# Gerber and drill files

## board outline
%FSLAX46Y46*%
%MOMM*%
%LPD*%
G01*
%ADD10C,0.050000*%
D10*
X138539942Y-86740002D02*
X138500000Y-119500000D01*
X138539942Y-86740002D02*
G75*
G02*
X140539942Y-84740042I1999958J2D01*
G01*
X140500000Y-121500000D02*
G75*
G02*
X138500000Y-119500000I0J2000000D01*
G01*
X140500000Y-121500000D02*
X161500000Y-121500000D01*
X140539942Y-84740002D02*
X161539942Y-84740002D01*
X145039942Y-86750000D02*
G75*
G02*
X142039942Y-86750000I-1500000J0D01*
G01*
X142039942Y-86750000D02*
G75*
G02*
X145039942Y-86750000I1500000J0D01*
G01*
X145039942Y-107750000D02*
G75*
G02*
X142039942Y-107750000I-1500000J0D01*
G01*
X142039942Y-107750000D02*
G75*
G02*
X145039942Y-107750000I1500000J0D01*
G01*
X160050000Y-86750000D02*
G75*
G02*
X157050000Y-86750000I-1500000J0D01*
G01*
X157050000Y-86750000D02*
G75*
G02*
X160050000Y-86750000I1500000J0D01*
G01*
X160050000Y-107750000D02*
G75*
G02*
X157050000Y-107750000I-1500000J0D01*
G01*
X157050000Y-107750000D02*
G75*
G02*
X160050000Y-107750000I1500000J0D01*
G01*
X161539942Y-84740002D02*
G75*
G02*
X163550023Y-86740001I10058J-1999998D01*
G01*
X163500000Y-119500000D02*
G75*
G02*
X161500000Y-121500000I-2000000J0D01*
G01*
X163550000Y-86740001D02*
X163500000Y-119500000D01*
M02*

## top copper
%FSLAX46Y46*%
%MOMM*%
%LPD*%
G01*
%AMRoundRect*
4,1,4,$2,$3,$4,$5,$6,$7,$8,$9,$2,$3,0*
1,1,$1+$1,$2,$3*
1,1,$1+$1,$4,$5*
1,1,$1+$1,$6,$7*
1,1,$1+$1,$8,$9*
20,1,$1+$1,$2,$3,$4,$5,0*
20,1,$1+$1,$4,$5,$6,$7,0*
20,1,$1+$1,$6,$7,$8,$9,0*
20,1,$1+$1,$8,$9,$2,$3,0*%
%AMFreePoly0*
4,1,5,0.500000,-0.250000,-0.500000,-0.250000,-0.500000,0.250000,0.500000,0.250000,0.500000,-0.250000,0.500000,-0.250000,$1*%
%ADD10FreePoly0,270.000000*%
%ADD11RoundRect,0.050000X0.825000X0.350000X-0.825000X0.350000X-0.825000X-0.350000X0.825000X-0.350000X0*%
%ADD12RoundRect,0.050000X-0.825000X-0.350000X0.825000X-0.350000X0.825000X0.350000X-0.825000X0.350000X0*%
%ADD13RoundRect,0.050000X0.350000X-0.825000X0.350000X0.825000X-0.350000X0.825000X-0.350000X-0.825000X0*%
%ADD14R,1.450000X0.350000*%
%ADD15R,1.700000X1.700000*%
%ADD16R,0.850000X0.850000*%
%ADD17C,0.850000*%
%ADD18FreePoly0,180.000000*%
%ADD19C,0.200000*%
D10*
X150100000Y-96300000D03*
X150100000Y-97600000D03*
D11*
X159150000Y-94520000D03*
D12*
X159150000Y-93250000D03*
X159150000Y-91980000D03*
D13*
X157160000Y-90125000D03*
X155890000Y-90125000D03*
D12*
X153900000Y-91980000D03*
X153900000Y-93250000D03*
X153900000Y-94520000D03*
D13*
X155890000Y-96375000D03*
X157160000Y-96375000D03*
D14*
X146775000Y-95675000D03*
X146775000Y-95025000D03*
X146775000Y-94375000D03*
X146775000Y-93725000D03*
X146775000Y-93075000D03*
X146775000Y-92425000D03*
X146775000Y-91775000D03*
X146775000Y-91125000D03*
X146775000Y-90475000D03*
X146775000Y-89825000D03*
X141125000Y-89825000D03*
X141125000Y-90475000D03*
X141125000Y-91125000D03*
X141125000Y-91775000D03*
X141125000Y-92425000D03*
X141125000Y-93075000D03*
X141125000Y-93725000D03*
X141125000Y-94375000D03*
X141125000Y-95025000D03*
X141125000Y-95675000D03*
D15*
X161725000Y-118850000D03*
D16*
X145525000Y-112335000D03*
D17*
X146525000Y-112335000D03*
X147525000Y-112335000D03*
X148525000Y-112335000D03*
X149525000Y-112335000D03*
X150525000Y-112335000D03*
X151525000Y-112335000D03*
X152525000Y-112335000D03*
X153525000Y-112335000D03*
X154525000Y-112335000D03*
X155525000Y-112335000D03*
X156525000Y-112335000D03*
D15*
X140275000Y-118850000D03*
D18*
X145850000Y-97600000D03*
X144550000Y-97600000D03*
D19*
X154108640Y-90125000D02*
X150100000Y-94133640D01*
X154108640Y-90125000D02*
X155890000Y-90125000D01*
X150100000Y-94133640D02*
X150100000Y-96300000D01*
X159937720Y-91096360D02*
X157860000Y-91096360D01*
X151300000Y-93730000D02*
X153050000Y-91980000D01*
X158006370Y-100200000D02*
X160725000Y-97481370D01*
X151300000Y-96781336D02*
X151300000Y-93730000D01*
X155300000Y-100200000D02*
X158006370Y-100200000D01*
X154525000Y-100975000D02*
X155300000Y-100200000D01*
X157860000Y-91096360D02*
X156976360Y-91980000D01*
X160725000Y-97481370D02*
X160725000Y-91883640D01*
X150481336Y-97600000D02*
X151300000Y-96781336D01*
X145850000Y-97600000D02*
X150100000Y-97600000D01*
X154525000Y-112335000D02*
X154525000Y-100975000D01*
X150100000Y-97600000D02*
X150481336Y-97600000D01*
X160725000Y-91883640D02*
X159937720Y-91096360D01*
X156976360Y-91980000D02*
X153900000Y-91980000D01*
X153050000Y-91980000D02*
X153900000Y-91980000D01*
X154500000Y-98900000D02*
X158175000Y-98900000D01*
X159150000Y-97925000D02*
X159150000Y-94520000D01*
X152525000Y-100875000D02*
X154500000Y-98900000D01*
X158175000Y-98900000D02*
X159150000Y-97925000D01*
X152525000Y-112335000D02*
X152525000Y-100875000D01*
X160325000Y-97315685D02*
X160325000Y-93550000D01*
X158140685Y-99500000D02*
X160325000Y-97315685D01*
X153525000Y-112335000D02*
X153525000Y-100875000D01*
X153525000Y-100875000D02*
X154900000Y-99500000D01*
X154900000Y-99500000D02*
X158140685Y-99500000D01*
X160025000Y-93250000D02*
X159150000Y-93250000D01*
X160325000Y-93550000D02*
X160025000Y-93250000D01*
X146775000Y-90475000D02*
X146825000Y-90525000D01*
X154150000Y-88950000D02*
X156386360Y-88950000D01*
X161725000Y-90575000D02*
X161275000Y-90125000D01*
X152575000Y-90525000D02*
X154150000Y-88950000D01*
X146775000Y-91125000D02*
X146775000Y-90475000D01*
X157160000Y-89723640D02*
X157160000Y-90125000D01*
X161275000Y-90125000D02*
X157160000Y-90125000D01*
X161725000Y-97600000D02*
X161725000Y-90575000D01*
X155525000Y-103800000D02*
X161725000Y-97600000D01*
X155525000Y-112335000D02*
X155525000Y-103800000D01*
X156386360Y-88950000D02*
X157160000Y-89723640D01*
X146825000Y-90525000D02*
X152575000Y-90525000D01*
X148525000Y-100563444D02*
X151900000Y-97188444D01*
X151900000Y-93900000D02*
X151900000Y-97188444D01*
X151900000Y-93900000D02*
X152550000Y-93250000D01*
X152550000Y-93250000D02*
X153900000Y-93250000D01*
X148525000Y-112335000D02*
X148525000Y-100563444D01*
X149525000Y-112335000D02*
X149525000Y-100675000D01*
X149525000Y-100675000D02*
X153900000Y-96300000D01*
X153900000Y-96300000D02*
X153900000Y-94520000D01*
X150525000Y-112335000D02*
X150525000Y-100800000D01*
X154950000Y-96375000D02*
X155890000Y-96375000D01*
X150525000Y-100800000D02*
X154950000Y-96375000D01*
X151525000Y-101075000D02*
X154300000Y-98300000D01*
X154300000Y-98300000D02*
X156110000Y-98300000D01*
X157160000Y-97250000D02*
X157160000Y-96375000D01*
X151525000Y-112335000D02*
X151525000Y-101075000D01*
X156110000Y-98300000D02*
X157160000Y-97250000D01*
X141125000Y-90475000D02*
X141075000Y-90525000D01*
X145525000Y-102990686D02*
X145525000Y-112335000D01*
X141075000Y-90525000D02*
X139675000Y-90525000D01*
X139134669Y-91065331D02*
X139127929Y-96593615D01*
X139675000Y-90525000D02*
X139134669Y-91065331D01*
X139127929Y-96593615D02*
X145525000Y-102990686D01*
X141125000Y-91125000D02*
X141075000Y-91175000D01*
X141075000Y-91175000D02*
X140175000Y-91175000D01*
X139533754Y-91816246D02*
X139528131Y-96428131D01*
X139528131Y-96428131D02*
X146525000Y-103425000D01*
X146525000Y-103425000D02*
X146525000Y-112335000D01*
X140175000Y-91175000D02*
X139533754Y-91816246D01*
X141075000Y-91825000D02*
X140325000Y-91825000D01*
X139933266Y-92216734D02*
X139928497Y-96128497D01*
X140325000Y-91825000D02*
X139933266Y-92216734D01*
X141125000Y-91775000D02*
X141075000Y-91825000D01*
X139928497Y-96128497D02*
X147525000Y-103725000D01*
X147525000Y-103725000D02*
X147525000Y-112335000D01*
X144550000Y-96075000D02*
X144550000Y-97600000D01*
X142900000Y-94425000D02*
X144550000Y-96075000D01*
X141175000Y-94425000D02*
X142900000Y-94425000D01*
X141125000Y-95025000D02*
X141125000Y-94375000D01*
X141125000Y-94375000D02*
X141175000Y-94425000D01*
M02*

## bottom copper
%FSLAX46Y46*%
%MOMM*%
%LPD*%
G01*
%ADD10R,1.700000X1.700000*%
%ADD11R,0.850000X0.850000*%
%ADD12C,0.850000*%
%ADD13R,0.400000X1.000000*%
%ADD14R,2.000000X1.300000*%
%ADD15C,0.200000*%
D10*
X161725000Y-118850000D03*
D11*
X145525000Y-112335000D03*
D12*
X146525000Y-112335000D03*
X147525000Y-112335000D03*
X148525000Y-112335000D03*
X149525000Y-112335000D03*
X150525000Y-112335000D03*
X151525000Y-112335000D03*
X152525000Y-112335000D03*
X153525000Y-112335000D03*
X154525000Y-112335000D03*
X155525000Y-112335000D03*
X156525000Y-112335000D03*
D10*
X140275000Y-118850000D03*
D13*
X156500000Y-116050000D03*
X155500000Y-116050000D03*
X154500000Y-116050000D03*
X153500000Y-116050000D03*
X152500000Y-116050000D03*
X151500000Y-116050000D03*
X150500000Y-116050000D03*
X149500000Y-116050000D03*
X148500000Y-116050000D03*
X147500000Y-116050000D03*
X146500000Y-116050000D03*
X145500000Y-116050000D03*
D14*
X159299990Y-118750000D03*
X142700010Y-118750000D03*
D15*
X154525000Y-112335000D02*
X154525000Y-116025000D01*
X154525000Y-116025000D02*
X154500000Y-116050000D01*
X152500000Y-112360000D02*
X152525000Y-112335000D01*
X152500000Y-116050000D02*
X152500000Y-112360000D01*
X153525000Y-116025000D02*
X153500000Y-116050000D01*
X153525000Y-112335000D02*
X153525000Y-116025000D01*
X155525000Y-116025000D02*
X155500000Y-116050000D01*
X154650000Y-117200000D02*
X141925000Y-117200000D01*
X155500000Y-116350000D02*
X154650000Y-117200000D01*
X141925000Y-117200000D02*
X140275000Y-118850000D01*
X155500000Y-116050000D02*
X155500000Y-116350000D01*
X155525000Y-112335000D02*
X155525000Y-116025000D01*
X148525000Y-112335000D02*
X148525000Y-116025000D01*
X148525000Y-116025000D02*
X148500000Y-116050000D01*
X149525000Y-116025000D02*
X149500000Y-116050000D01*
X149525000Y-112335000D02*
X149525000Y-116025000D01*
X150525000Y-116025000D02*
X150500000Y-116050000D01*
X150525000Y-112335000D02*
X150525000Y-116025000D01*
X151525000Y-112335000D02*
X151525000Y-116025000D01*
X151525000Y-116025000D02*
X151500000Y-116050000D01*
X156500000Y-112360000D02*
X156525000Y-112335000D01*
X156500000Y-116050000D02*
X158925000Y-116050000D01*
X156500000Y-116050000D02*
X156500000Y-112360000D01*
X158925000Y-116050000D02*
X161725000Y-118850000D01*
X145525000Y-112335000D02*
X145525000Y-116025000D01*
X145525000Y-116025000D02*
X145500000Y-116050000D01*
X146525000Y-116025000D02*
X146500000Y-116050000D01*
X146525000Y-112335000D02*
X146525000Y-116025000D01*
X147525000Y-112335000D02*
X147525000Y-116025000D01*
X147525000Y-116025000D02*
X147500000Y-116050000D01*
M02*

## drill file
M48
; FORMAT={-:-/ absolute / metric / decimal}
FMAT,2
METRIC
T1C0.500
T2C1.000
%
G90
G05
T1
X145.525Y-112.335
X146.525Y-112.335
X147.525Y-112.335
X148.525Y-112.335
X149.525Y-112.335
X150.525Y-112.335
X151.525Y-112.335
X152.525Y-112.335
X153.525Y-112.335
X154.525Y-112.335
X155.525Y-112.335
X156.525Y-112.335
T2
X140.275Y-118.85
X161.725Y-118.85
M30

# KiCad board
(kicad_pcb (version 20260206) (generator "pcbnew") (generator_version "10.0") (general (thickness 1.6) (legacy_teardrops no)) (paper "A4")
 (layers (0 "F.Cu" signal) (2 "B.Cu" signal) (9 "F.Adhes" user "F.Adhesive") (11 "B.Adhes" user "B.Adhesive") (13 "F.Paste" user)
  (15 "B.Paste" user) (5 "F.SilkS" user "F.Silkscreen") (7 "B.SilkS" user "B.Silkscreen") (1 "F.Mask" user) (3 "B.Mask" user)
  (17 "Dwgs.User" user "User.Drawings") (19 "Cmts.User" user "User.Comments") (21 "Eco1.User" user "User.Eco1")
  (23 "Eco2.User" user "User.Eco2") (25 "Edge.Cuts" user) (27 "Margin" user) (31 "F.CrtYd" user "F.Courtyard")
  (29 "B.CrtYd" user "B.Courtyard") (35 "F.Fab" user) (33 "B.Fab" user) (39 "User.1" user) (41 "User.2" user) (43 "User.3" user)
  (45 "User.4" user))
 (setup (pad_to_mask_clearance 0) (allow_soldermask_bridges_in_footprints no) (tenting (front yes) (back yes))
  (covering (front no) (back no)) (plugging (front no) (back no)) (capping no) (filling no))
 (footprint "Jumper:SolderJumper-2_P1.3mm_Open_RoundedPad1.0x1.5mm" (layer "F.Cu") (at 150.1 96.95 -90)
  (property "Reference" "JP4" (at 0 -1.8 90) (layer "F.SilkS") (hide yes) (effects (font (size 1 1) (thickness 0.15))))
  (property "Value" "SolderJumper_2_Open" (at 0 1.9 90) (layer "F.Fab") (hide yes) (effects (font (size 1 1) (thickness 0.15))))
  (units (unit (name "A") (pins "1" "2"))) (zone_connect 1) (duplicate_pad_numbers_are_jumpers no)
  (pad "1" smd custom (at -0.65 0 270) (size 1 0.5) (layers "F.Cu" "F.Mask") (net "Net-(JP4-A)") (zone_connect 2) (thermal_bridge_angle 45)
   (options (clearance outline) (anchor rect)) (primitives))
  (pad "2" smd custom (at 0.65 0 270) (size 1 0.5) (layers "F.Cu" "F.Mask") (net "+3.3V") (zone_connect 2) (thermal_bridge_angle 45)
   (options (clearance outline) (anchor rect)) (primitives)))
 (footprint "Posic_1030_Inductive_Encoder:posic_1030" (layer "F.Cu") (at 160.025 93.25 180)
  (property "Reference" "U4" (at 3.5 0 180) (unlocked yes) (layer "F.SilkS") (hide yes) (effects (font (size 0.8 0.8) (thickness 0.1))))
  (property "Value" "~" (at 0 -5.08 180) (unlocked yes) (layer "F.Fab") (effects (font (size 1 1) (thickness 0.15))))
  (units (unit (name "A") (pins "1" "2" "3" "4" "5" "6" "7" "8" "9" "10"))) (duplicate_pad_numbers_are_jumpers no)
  (pad "1" smd roundrect (at 0.875 -1.27 180) (size 1.75 0.8) (layers "F.Cu" "F.Mask" "F.Paste") (roundrect_rratio 0.0625) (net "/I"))
  (pad "2" smd roundrect (at 0.875 0) (size 1.75 0.8) (layers "F.Cu" "F.Mask" "F.Paste") (roundrect_rratio 0.0625) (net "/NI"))
  (pad "3" smd roundrect (at 0.875 1.27) (size 1.75 0.8) (layers "F.Cu" "F.Mask" "F.Paste") (roundrect_rratio 0.0625)
   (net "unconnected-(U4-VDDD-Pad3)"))
  (pad "4" smd roundrect (at 2.865 3.125 90) (size 1.75 0.8) (layers "F.Cu" "F.Mask" "F.Paste") (roundrect_rratio 0.0625) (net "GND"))
  (pad "5" smd roundrect (at 4.135 3.125 90) (size 1.75 0.8) (layers "F.Cu" "F.Mask" "F.Paste") (roundrect_rratio 0.0625)
   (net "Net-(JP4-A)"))
  (pad "6" smd roundrect (at 6.125 1.27) (size 1.75 0.8) (layers "F.Cu" "F.Mask" "F.Paste") (roundrect_rratio 0.0625) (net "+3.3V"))
  (pad "7" smd roundrect (at 6.125 0) (size 1.75 0.8) (layers "F.Cu" "F.Mask" "F.Paste") (roundrect_rratio 0.0625) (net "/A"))
  (pad "8" smd roundrect (at 6.125 -1.27) (size 1.75 0.8) (layers "F.Cu" "F.Mask" "F.Paste") (roundrect_rratio 0.0625) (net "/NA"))
  (pad "9" smd roundrect (at 4.135 -3.125 90) (size 1.75 0.8) (layers "F.Cu" "F.Mask" "F.Paste") (roundrect_rratio 0.0625) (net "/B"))
  (pad "10" smd roundrect (at 2.865 -3.125 90) (size 1.75 0.8) (layers "F.Cu" "F.Mask" "F.Paste") (roundrect_rratio 0.0625) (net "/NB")))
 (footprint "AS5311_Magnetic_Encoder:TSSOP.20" (layer "F.Cu") (at 143.95 92.75 90)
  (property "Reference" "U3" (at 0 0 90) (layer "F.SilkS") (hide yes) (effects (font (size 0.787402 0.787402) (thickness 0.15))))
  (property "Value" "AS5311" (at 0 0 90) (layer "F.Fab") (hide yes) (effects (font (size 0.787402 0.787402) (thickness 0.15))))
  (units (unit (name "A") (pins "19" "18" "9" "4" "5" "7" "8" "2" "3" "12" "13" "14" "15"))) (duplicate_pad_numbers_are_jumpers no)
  (pad "1" smd rect (at -2.925 2.825 90) (size 0.35 1.45) (layers "F.Cu" "F.Mask" "F.Paste") (solder_mask_margin 0.102))
  (pad "2" smd rect (at -2.275 2.825 90) (size 0.35 1.45) (layers "F.Cu" "F.Mask" "F.Paste") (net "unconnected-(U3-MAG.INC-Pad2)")
   (solder_mask_margin 0.102))
  (pad "3" smd rect (at -1.625 2.825 90) (size 0.35 1.45) (layers "F.Cu" "F.Mask" "F.Paste") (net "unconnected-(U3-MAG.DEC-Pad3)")
   (solder_mask_margin 0.102))
  (pad "4" smd rect (at -0.975 2.825 90) (size 0.35 1.45) (layers "F.Cu" "F.Mask" "F.Paste") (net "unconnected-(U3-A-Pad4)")
   (solder_mask_margin 0.102))
  (pad "5" smd rect (at -0.325 2.825 90) (size 0.35 1.45) (layers "F.Cu" "F.Mask" "F.Paste") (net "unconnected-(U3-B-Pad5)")
   (solder_mask_margin 0.102))
  (pad "6" smd rect (at 0.325 2.825 90) (size 0.35 1.45) (layers "F.Cu" "F.Mask" "F.Paste") (solder_mask_margin 0.102))
  (pad "7" smd rect (at 0.975 2.825 90) (size 0.35 1.45) (layers "F.Cu" "F.Mask" "F.Paste") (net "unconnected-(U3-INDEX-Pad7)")
   (solder_mask_margin 0.102))
  (pad "8" smd rect (at 1.625 2.825 90) (size 0.35 1.45) (layers "F.Cu" "F.Mask" "F.Paste") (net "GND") (solder_mask_margin 0.102))
  (pad "9" smd rect (at 2.275 2.825 90) (size 0.35 1.45) (layers "F.Cu" "F.Mask" "F.Paste") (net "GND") (solder_mask_margin 0.102))
  (pad "10" smd rect (at 2.925 2.825 90) (size 0.35 1.45) (layers "F.Cu" "F.Mask" "F.Paste") (solder_mask_margin 0.102))
  (pad "11" smd rect (at 2.925 -2.825 90) (size 0.35 1.45) (layers "F.Cu" "F.Mask" "F.Paste") (solder_mask_margin 0.102))
  (pad "12" smd rect (at 2.275 -2.825 90) (size 0.35 1.45) (layers "F.Cu" "F.Mask" "F.Paste") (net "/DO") (solder_mask_margin 0.102))
  (pad "13" smd rect (at 1.625 -2.825 90) (size 0.35 1.45) (layers "F.Cu" "F.Mask" "F.Paste") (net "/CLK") (solder_mask_margin 0.102))
  (pad "14" smd rect (at 0.975 -2.825 90) (size 0.35 1.45) (layers "F.Cu" "F.Mask" "F.Paste") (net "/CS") (solder_mask_margin 0.102))
  (pad "15" smd rect (at 0.325 -2.825 90) (size 0.35 1.45) (layers "F.Cu" "F.Mask" "F.Paste") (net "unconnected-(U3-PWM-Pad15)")
   (solder_mask_margin 0.102))
  (pad "16" smd rect (at -0.325 -2.825 90) (size 0.35 1.45) (layers "F.Cu" "F.Mask" "F.Paste") (solder_mask_margin 0.102))
  (pad "17" smd rect (at -0.975 -2.825 90) (size 0.35 1.45) (layers "F.Cu" "F.Mask" "F.Paste") (solder_mask_margin 0.102))
  (pad "18" smd rect (at -1.625 -2.825 90) (size 0.35 1.45) (layers "F.Cu" "F.Mask" "F.Paste") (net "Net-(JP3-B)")
   (solder_mask_margin 0.102))
  (pad "19" smd rect (at -2.275 -2.825 90) (size 0.35 1.45) (layers "F.Cu" "F.Mask" "F.Paste") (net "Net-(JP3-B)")
   (solder_mask_margin 0.102))
  (pad "20" smd rect (at -2.925 -2.825 90) (size 0.35 1.45) (layers "F.Cu" "F.Mask" "F.Paste") (solder_mask_margin 0.102)))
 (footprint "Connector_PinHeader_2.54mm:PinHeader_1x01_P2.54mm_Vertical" (layer "F.Cu") (at 161.725 118.85)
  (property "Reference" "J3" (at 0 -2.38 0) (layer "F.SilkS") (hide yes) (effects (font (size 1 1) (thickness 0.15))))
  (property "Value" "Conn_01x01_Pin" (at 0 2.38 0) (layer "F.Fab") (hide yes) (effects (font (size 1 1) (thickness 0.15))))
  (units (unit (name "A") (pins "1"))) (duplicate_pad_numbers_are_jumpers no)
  (pad "1" thru_hole rect (at 0 0) (size 1.7 1.7) (drill 1) (layers "*.Cu" "*.Mask") (remove_unused_layers no) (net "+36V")))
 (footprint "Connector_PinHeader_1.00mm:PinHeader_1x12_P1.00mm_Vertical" (layer "F.Cu") (at 145.525 112.335 90)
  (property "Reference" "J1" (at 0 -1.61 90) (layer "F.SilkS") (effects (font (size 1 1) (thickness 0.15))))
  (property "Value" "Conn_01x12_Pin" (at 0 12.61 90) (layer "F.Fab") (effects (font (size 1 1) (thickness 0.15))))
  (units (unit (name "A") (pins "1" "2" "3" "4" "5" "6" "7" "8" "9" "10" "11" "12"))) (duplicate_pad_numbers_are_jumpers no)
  (pad "1" thru_hole rect (at 0 0 90) (size 0.85 0.85) (drill 0.5) (layers "*.Cu" "*.Mask") (remove_unused_layers no) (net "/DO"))
  (pad "2" thru_hole circle (at 0 1 90) (size 0.85 0.85) (drill 0.5) (layers "*.Cu" "*.Mask") (remove_unused_layers no) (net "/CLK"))
  (pad "3" thru_hole circle (at 0 2 90) (size 0.85 0.85) (drill 0.5) (layers "*.Cu" "*.Mask") (remove_unused_layers no) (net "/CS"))
  (pad "4" thru_hole circle (at 0 3 90) (size 0.85 0.85) (drill 0.5) (layers "*.Cu" "*.Mask") (remove_unused_layers no) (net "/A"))
  (pad "5" thru_hole circle (at 0 4 90) (size 0.85 0.85) (drill 0.5) (layers "*.Cu" "*.Mask") (remove_unused_layers no) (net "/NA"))
  (pad "6" thru_hole circle (at 0 5 90) (size 0.85 0.85) (drill 0.5) (layers "*.Cu" "*.Mask") (remove_unused_layers no) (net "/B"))
  (pad "7" thru_hole circle (at 0 6 90) (size 0.85 0.85) (drill 0.5) (layers "*.Cu" "*.Mask") (remove_unused_layers no) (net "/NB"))
  (pad "8" thru_hole circle (at 0 7 90) (size 0.85 0.85) (drill 0.5) (layers "*.Cu" "*.Mask") (remove_unused_layers no) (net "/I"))
  (pad "9" thru_hole circle (at 0 8 90) (size 0.85 0.85) (drill 0.5) (layers "*.Cu" "*.Mask") (remove_unused_layers no) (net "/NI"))
  (pad "10" thru_hole circle (at 0 9 90) (size 0.85 0.85) (drill 0.5) (layers "*.Cu" "*.Mask") (remove_unused_layers no) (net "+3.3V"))
  (pad "11" thru_hole circle (at 0 10 90) (size 0.85 0.85) (drill 0.5) (layers "*.Cu" "*.Mask") (remove_unused_layers no) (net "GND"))
  (pad "12" thru_hole circle (at 0 11 90) (size 0.85 0.85) (drill 0.5) (layers "*.Cu" "*.Mask") (remove_unused_layers no) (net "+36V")))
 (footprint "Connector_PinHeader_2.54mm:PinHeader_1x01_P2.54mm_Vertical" (layer "F.Cu") (at 140.275 118.85)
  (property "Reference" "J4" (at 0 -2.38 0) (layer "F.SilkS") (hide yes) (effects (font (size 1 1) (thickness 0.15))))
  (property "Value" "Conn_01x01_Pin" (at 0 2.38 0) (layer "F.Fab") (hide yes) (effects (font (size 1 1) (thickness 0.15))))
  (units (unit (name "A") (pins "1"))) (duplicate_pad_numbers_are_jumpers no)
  (pad "1" thru_hole rect (at 0 0) (size 1.7 1.7) (drill 1) (layers "*.Cu" "*.Mask") (remove_unused_layers no) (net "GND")))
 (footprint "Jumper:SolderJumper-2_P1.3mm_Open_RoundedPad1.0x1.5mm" (layer "F.Cu") (at 145.2 97.6 180)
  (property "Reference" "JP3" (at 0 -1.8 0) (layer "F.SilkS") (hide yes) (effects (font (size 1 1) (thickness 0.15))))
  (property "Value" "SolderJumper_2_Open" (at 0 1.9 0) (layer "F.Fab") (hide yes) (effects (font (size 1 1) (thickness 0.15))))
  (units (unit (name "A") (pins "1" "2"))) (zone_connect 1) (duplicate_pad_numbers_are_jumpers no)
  (pad "1" smd custom (at -0.65 0 180) (size 1 0.5) (layers "F.Cu" "F.Mask") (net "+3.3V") (zone_connect 2) (thermal_bridge_angle 45)
   (options (clearance outline) (anchor rect)) (primitives))
  (pad "2" smd custom (at 0.65 0 180) (size 1 0.5) (layers "F.Cu" "F.Mask") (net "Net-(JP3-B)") (zone_connect 2) (thermal_bridge_angle 45)
   (options (clearance outline) (anchor rect)) (primitives)))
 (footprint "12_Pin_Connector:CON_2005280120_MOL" (layer "B.Cu") (at 151 118.5 180)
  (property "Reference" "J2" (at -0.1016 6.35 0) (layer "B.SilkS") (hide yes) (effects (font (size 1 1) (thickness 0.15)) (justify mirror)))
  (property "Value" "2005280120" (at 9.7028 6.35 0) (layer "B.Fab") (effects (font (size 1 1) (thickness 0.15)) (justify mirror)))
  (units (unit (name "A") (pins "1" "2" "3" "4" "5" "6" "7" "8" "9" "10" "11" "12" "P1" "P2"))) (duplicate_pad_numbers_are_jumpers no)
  (pad "1" smd rect (at -5.5 2.45 180) (size 0.4 1) (layers "B.Cu" "B.Mask" "B.Paste") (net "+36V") (solder_mask_margin 0.102))
  (pad "2" smd rect (at -4.5 2.45 180) (size 0.4 1) (layers "B.Cu" "B.Mask" "B.Paste") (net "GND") (solder_mask_margin 0.102))
  (pad "3" smd rect (at -3.5 2.45 180) (size 0.4 1) (layers "B.Cu" "B.Mask" "B.Paste") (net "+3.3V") (solder_mask_margin 0.102))
  (pad "4" smd rect (at -2.5 2.45 180) (size 0.4 1) (layers "B.Cu" "B.Mask" "B.Paste") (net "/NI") (solder_mask_margin 0.102))
  (pad "5" smd rect (at -1.5 2.45 180) (size 0.4 1) (layers "B.Cu" "B.Mask" "B.Paste") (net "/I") (solder_mask_margin 0.102))
  (pad "6" smd rect (at -0.5 2.45 180) (size 0.4 1) (layers "B.Cu" "B.Mask" "B.Paste") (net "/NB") (solder_mask_margin 0.102))
  (pad "7" smd rect (at 0.5 2.45 180) (size 0.4 1) (layers "B.Cu" "B.Mask" "B.Paste") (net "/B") (solder_mask_margin 0.102))
  (pad "8" smd rect (at 1.5 2.45 180) (size 0.4 1) (layers "B.Cu" "B.Mask" "B.Paste") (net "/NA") (solder_mask_margin 0.102))
  (pad "9" smd rect (at 2.5 2.45 180) (size 0.4 1) (layers "B.Cu" "B.Mask" "B.Paste") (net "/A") (solder_mask_margin 0.102))
  (pad "10" smd rect (at 3.5 2.45 180) (size 0.4 1) (layers "B.Cu" "B.Mask" "B.Paste") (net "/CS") (solder_mask_margin 0.102))
  (pad "11" smd rect (at 4.5 2.45 180) (size 0.4 1) (layers "B.Cu" "B.Mask" "B.Paste") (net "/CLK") (solder_mask_margin 0.102))
  (pad "12" smd rect (at 5.5 2.45 180) (size 0.4 1) (layers "B.Cu" "B.Mask" "B.Paste") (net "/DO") (solder_mask_margin 0.102))
  (pad "P1" smd rect (at -8.29999 -0.25 180) (size 2 1.3) (layers "B.Cu" "B.Mask" "B.Paste") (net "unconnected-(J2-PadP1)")
   (solder_mask_margin 0.102))
  (pad "P2" smd rect (at 8.29999 -0.25 180) (size 2 1.3) (layers "B.Cu" "B.Mask" "B.Paste") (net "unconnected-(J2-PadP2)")
   (solder_mask_margin 0.102)))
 (gr_line (start 138.539942 86.740002) (end 138.5 119.5) (stroke (width 0.05) (type solid)) (layer "Edge.Cuts"))
 (gr_arc (start 138.539942 86.740002) (mid 139.125728 85.325788) (end 140.539942 84.740002) (stroke (width 0.05) (type default))
  (layer "Edge.Cuts"))
 (gr_arc (start 140.5 121.5) (mid 139.085786 120.914214) (end 138.5 119.5) (stroke (width 0.05) (type default)) (layer "Edge.Cuts"))
 (gr_line (start 140.5 121.5) (end 161.5 121.5) (stroke (width 0.05) (type solid)) (layer "Edge.Cuts"))
 (gr_line (start 140.539942 84.740002) (end 161.539942 84.740002) (stroke (width 0.05) (type solid)) (layer "Edge.Cuts"))
 (gr_circle (center 143.539942 86.75) (end 145.039942 86.75) (stroke (width 0.05) (type solid)) (fill no) (layer "Edge.Cuts"))
 (gr_circle (center 143.539942 107.75) (end 145.039942 107.75) (stroke (width 0.05) (type solid)) (fill no) (layer "Edge.Cuts"))
 (gr_circle (center 158.55 86.75) (end 160.05 86.75) (stroke (width 0.05) (type solid)) (fill no) (layer "Edge.Cuts"))
 (gr_circle (center 158.55 107.75) (end 160.05 107.75) (stroke (width 0.05) (type solid)) (fill no) (layer "Edge.Cuts"))
 (gr_arc (start 161.539942 84.740002) (mid 162.96067 85.322219) (end 163.550024 86.740001) (stroke (width 0.05) (type default))
  (layer "Edge.Cuts"))
 (gr_arc (start 163.5 119.5) (mid 162.914214 120.914214) (end 161.5 121.5) (stroke (width 0.05) (type default)) (layer "Edge.Cuts"))
 (gr_line (start 163.55 86.740001) (end 163.5 119.5) (stroke (width 0.05) (type solid)) (layer "Edge.Cuts"))
 (segment (start 154.10864 90.125) (end 150.1 94.13364) (width 0.2) (layer "F.Cu") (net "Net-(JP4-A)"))
 (segment (start 154.10864 90.125) (end 155.89 90.125) (width 0.2) (layer "F.Cu") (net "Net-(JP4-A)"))
 (segment (start 150.1 94.13364) (end 150.1 96.3) (width 0.2) (layer "F.Cu") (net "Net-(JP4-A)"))
 (segment (start 159.93772 91.09636) (end 157.86 91.09636) (width 0.2) (layer "F.Cu") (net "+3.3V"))
 (segment (start 151.3 93.73) (end 153.05 91.98) (width 0.2) (layer "F.Cu") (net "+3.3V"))
 (segment (start 158.00637 100.2) (end 160.725 97.48137) (width 0.2) (layer "F.Cu") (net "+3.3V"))
 (segment (start 151.3 96.781336) (end 151.3 93.73) (width 0.2) (layer "F.Cu") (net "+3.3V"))
 (segment (start 155.3 100.2) (end 158.00637 100.2) (width 0.2) (layer "F.Cu") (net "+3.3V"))
 (segment (start 154.525 100.975) (end 155.3 100.2) (width 0.2) (layer "F.Cu") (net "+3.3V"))
 (segment (start 157.86 91.09636) (end 156.97636 91.98) (width 0.2) (layer "F.Cu") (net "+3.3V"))
 (segment (start 160.725 97.48137) (end 160.725 91.88364) (width 0.2) (layer "F.Cu") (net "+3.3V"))
 (segment (start 150.481336 97.6) (end 151.3 96.781336) (width 0.2) (layer "F.Cu") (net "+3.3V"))
 (segment (start 145.85 97.6) (end 150.1 97.6) (width 0.2) (layer "F.Cu") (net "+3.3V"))
 (segment (start 154.525 112.335) (end 154.525 100.975) (width 0.2) (layer "F.Cu") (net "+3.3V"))
 (segment (start 150.1 97.6) (end 150.481336 97.6) (width 0.2) (layer "F.Cu") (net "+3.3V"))
 (segment (start 160.725 91.88364) (end 159.93772 91.09636) (width 0.2) (layer "F.Cu") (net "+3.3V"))
 (segment (start 156.97636 91.98) (end 153.9 91.98) (width 0.2) (layer "F.Cu") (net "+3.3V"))
 (segment (start 153.05 91.98) (end 153.9 91.98) (width 0.2) (layer "F.Cu") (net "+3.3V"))
 (segment (start 154.525 112.335) (end 154.525 116.025) (width 0.2) (layer "B.Cu") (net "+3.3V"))
 (segment (start 154.525 116.025) (end 154.5 116.05) (width 0.2) (layer "B.Cu") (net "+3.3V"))
 (segment (start 154.5 98.9) (end 158.175 98.9) (width 0.2) (layer "F.Cu") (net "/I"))
 (segment (start 159.15 97.925) (end 159.15 94.52) (width 0.2) (layer "F.Cu") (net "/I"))
 (segment (start 152.525 100.875) (end 154.5 98.9) (width 0.2) (layer "F.Cu") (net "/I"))
 (segment (start 158.175 98.9) (end 159.15 97.925) (width 0.2) (layer "F.Cu") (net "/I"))
 (segment (start 152.525 112.335) (end 152.525 100.875) (width 0.2) (layer "F.Cu") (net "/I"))
 (segment (start 152.5 112.36) (end 152.525 112.335) (width 0.2) (layer "B.Cu") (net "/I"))
 (segment (start 152.5 116.05) (end 152.5 112.36) (width 0.2) (layer "B.Cu") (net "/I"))
 (segment (start 160.325 97.315685) (end 160.325 93.55) (width 0.2) (layer "F.Cu") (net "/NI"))
 (segment (start 158.140685 99.5) (end 160.325 97.315685) (width 0.2) (layer "F.Cu") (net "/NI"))
 (segment (start 153.525 112.335) (end 153.525 100.875) (width 0.2) (layer "F.Cu") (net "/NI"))
 (segment (start 153.525 100.875) (end 154.9 99.5) (width 0.2) (layer "F.Cu") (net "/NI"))
 (segment (start 154.9 99.5) (end 158.140685 99.5) (width 0.2) (layer "F.Cu") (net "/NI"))
 (segment (start 160.025 93.25) (end 159.15 93.25) (width 0.2) (layer "F.Cu") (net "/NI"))
 (segment (start 160.325 93.55) (end 160.025 93.25) (width 0.2) (layer "F.Cu") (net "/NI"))
 (segment (start 153.525 116.025) (end 153.5 116.05) (width 0.2) (layer "B.Cu") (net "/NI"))
 (segment (start 153.525 112.335) (end 153.525 116.025) (width 0.2) (layer "B.Cu") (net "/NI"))
 (segment (start 146.775 90.475) (end 146.825 90.525) (width 0.2) (layer "F.Cu") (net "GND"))
 (segment (start 154.15 88.95) (end 156.38636 88.95) (width 0.2) (layer "F.Cu") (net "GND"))
 (segment (start 161.725 90.575) (end 161.275 90.125) (width 0.2) (layer "F.Cu") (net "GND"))
 (segment (start 152.575 90.525) (end 154.15 88.95) (width 0.2) (layer "F.Cu") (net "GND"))
 (segment (start 146.775 91.125) (end 146.775 90.475) (width 0.2) (layer "F.Cu") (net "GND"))
 (segment (start 157.16 89.72364) (end 157.16 90.125) (width 0.2) (layer "F.Cu") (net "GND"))
 (segment (start 161.275 90.125) (end 157.16 90.125) (width 0.2) (layer "F.Cu") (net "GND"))
 (segment (start 161.725 97.6) (end 161.725 90.575) (width 0.2) (layer "F.Cu") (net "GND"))
 (segment (start 155.525 103.8) (end 161.725 97.6) (width 0.2) (layer "F.Cu") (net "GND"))
 (segment (start 155.525 112.335) (end 155.525 103.8) (width 0.2) (layer "F.Cu") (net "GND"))
 (segment (start 156.38636 88.95) (end 157.16 89.72364) (width 0.2) (layer "F.Cu") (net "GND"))
 (segment (start 146.825 90.525) (end 152.575 90.525) (width 0.2) (layer "F.Cu") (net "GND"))
 (segment (start 155.525 116.025) (end 155.5 116.05) (width 0.2) (layer "B.Cu") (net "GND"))
 (segment (start 154.65 117.2) (end 141.925 117.2) (width 0.2) (layer "B.Cu") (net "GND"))
 (segment (start 155.5 116.35) (end 154.65 117.2) (width 0.2) (layer "B.Cu") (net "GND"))
 (segment (start 141.925 117.2) (end 140.275 118.85) (width 0.2) (layer "B.Cu") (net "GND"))
 (segment (start 155.5 116.05) (end 155.5 116.35) (width 0.2) (layer "B.Cu") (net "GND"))
 (segment (start 155.525 112.335) (end 155.525 116.025) (width 0.2) (layer "B.Cu") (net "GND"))
 (segment (start 148.525 100.563444) (end 151.9 97.188444) (width 0.2) (layer "F.Cu") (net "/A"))
 (segment (start 151.9 93.9) (end 151.9 97.188444) (width 0.2) (layer "F.Cu") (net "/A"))
 (segment (start 151.9 93.9) (end 152.55 93.25) (width 0.2) (layer "F.Cu") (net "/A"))
 (segment (start 152.55 93.25) (end 153.9 93.25) (width 0.2) (layer "F.Cu") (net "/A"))
 (segment (start 148.525 112.335) (end 148.525 100.563444) (width 0.2) (layer "F.Cu") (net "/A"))
 (segment (start 148.525 112.335) (end 148.525 116.025) (width 0.2) (layer "B.Cu") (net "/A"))
 (segment (start 148.525 116.025) (end 148.5 116.05) (width 0.2) (layer "B.Cu") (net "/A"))
 (segment (start 149.525 112.335) (end 149.525 100.675) (width 0.2) (layer "F.Cu") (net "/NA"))
 (segment (start 149.525 100.675) (end 153.9 96.3) (width 0.2) (layer "F.Cu") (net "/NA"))
 (segment (start 153.9 96.3) (end 153.9 94.52) (width 0.2) (layer "F.Cu") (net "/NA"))
 (segment (start 149.525 116.025) (end 149.5 116.05) (width 0.2) (layer "B.Cu") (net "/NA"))
 (segment (start 149.525 112.335) (end 149.525 116.025) (width 0.2) (layer "B.Cu") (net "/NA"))
 (segment (start 150.525 112.335) (end 150.525 100.8) (width 0.2) (layer "F.Cu") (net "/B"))
 (segment (start 154.95 96.375) (end 155.89 96.375) (width 0.2) (layer "F.Cu") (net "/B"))
 (segment (start 150.525 100.8) (end 154.95 96.375) (width 0.2) (layer "F.Cu") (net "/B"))
 (segment (start 150.525 116.025) (end 150.5 116.05) (width 0.2) (layer "B.Cu") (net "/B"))
 (segment (start 150.525 112.335) (end 150.525 116.025) (width 0.2) (layer "B.Cu") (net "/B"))
 (segment (start 151.525 101.075) (end 154.3 98.3) (width 0.2) (layer "F.Cu") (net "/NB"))
 (segment (start 154.3 98.3) (end 156.11 98.3) (width 0.2) (layer "F.Cu") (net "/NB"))
 (segment (start 157.16 97.25) (end 157.16 96.375) (width 0.2) (layer "F.Cu") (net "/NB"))
 (segment (start 151.525 112.335) (end 151.525 101.075) (width 0.2) (layer "F.Cu") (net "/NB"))
 (segment (start 156.11 98.3) (end 157.16 97.25) (width 0.2) (layer "F.Cu") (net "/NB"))
 (segment (start 151.525 112.335) (end 151.525 116.025) (width 0.2) (layer "B.Cu") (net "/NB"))
 (segment (start 151.525 116.025) (end 151.5 116.05) (width 0.2) (layer "B.Cu") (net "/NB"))
 (segment (start 156.5 112.36) (end 156.525 112.335) (width 0.2) (layer "B.Cu") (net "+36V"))
 (segment (start 156.5 116.05) (end 158.925 116.05) (width 0.2) (layer "B.Cu") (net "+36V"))
 (segment (start 156.5 116.05) (end 156.5 112.36) (width 0.2) (layer "B.Cu") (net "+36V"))
 (segment (start 158.925 116.05) (end 161.725 118.85) (width 0.2) (layer "B.Cu") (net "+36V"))
 (segment (start 141.125 90.475) (end 141.075 90.525) (width 0.2) (layer "F.Cu") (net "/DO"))
 (segment (start 145.525 102.990686) (end 145.525 112.335) (width 0.2) (layer "F.Cu") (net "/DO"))
 (segment (start 141.075 90.525) (end 139.675 90.525) (width 0.2) (layer "F.Cu") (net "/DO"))
 (segment (start 139.134669 91.065331) (end 139.127929 96.593615) (width 0.2) (layer "F.Cu") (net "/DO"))
 (segment (start 139.675 90.525) (end 139.134669 91.065331) (width 0.2) (layer "F.Cu") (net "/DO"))
 (segment (start 139.127929 96.593615) (end 145.525 102.990686) (width 0.2) (layer "F.Cu") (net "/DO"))
 (segment (start 145.525 112.335) (end 145.525 116.025) (width 0.2) (layer "B.Cu") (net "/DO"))
 (segment (start 145.525 116.025) (end 145.5 116.05) (width 0.2) (layer "B.Cu") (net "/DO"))
 (segment (start 141.125 91.125) (end 141.075 91.175) (width 0.2) (layer "F.Cu") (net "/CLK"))
 (segment (start 141.075 91.175) (end 140.175 91.175) (width 0.2) (layer "F.Cu") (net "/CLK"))
 (segment (start 139.533754 91.816246) (end 139.528131 96.428131) (width 0.2) (layer "F.Cu") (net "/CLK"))
 (segment (start 139.528131 96.428131) (end 146.525 103.425) (width 0.2) (layer "F.Cu") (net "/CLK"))
 (segment (start 146.525 103.425) (end 146.525 112.335) (width 0.2) (layer "F.Cu") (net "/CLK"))
 (segment (start 140.175 91.175) (end 139.533754 91.816246) (width 0.2) (layer "F.Cu") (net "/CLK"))
 (segment (start 146.525 116.025) (end 146.5 116.05) (width 0.2) (layer "B.Cu") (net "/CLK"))
 (segment (start 146.525 112.335) (end 146.525 116.025) (width 0.2) (layer "B.Cu") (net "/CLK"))
 (segment (start 141.075 91.825) (end 140.325 91.825) (width 0.2) (layer "F.Cu") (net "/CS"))
 (segment (start 139.933266 92.216734) (end 139.928497 96.128497) (width 0.2) (layer "F.Cu") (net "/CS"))
 (segment (start 140.325 91.825) (end 139.933266 92.216734) (width 0.2) (layer "F.Cu") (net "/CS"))
 (segment (start 141.125 91.775) (end 141.075 91.825) (width 0.2) (layer "F.Cu") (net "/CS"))
 (segment (start 139.928497 96.128497) (end 147.525 103.725) (width 0.2) (layer "F.Cu") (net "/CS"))
 (segment (start 147.525 103.725) (end 147.525 112.335) (width 0.2) (layer "F.Cu") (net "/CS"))
 (segment (start 147.525 112.335) (end 147.525 116.025) (width 0.2) (layer "B.Cu") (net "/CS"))
 (segment (start 147.525 116.025) (end 147.5 116.05) (width 0.2) (layer "B.Cu") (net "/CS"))
 (segment (start 144.55 96.075) (end 144.55 97.6) (width 0.2) (layer "F.Cu") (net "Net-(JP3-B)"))
 (segment (start 142.9 94.425) (end 144.55 96.075) (width 0.2) (layer "F.Cu") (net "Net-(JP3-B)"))
 (segment (start 141.175 94.425) (end 142.9 94.425) (width 0.2) (layer "F.Cu") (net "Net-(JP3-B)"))
 (segment (start 141.125 95.025) (end 141.125 94.375) (width 0.2) (layer "F.Cu") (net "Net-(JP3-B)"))
 (segment (start 141.125 94.375) (end 141.175 94.425) (width 0.2) (layer "F.Cu") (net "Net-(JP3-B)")))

